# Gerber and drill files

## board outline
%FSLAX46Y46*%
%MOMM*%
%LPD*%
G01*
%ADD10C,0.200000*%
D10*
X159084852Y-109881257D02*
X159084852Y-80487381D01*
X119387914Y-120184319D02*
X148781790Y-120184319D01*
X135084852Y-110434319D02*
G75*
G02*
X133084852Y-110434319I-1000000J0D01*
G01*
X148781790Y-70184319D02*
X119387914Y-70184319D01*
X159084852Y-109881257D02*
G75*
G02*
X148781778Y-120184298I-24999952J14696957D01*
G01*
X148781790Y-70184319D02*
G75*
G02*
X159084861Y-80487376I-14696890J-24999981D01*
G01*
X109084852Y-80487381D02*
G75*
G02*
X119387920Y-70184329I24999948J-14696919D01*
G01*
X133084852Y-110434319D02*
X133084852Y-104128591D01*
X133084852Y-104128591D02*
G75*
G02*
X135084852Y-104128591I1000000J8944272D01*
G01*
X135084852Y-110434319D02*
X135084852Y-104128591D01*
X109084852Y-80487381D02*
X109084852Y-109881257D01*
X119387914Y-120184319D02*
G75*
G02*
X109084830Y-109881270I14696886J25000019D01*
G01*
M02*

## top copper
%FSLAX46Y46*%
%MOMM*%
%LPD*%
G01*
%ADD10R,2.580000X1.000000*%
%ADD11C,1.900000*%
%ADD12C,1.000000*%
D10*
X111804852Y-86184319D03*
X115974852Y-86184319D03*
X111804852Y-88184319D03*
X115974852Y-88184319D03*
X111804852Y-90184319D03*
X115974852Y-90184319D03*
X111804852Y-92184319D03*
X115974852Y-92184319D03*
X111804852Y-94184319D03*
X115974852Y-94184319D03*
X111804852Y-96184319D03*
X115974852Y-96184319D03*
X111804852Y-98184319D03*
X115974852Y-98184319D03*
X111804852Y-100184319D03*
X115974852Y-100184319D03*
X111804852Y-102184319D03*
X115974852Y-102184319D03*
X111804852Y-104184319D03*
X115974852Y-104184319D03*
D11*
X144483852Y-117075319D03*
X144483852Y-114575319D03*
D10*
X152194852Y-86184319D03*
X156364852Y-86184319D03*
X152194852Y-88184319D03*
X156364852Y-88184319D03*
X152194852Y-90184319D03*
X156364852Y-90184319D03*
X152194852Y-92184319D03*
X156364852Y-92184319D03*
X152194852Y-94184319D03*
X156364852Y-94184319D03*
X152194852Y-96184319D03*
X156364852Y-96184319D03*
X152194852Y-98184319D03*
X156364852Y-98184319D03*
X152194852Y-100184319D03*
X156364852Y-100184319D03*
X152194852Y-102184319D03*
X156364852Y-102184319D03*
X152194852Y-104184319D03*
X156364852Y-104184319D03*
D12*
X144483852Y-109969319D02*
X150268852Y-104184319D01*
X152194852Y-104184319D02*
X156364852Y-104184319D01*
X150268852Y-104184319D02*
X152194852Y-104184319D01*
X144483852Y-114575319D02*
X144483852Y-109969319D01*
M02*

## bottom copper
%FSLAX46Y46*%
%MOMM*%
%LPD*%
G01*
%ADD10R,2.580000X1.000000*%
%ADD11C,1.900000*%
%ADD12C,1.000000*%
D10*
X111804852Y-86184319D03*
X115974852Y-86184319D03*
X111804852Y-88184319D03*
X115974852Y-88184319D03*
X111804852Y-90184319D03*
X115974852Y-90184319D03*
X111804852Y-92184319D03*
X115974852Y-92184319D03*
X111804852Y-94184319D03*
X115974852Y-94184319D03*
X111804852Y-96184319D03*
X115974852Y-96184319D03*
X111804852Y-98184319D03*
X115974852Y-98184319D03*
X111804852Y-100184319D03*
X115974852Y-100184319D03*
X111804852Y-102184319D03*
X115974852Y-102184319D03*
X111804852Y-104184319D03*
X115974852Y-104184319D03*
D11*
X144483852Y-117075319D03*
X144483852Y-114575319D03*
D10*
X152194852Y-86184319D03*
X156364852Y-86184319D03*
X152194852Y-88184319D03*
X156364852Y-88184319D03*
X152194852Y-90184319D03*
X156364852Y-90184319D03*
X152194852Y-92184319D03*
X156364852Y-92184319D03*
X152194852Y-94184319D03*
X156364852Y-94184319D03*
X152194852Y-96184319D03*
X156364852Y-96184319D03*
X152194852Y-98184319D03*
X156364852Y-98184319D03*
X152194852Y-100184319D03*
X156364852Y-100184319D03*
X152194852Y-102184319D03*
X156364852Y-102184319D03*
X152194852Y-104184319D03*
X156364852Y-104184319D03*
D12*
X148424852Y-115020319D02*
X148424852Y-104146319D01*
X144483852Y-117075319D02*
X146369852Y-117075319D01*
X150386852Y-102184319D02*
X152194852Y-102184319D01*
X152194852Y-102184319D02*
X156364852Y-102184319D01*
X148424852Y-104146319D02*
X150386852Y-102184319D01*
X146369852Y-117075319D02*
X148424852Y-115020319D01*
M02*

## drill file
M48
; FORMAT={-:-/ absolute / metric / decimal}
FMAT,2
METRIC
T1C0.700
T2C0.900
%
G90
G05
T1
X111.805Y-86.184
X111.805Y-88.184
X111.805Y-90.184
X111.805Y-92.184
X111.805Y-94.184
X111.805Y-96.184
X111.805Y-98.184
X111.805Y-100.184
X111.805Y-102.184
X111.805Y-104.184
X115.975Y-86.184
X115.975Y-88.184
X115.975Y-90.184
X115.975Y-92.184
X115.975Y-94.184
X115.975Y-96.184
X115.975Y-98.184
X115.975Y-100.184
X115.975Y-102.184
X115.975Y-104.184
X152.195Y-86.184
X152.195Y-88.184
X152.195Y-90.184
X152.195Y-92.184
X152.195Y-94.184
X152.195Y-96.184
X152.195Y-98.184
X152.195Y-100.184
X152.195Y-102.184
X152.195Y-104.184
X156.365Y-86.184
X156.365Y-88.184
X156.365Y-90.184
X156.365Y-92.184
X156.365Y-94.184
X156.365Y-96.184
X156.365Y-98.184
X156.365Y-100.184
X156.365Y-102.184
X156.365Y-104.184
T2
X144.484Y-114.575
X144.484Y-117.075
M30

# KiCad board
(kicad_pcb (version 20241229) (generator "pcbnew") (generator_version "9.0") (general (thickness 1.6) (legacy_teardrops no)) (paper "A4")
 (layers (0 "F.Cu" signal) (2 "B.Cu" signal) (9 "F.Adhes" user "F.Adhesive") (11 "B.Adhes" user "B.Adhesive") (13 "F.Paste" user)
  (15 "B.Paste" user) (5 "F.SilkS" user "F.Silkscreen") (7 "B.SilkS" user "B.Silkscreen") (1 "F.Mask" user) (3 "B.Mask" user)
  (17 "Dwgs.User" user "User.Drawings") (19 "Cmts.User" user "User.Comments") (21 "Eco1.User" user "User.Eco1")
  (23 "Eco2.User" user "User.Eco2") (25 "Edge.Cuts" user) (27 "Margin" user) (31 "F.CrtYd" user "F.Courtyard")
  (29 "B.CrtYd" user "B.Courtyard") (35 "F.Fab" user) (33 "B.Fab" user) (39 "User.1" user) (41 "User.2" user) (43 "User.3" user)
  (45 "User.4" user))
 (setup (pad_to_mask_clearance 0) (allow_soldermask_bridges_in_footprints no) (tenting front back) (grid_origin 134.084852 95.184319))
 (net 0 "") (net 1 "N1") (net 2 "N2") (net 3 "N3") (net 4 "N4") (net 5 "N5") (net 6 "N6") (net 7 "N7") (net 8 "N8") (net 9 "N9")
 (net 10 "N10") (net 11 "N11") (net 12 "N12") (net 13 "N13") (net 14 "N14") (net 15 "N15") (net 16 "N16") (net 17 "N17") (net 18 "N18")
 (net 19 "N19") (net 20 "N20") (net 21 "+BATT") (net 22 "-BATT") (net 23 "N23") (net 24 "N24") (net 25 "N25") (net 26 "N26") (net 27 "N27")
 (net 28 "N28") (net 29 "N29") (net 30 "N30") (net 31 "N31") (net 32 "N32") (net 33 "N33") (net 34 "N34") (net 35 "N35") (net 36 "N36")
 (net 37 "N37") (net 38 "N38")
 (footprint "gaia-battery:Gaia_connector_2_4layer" (layer "F.Cu") (at 113.889852 95.184319)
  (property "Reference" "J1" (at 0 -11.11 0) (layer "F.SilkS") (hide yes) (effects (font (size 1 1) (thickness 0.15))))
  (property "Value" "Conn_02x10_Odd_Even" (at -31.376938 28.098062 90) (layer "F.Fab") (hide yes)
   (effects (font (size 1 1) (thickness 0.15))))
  (pad "1" thru_hole rect (at -2.085 -9) (size 2.58 1) (drill 0.7) (layers "*.Cu" "*.Mask") (remove_unused_layers no) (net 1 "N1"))
  (pad "2" thru_hole rect (at 2.085 -9) (size 2.58 1) (drill 0.7) (layers "*.Cu" "*.Mask") (remove_unused_layers no) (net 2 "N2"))
  (pad "3" thru_hole rect (at -2.085 -7) (size 2.58 1) (drill 0.7) (layers "*.Cu" "*.Mask") (remove_unused_layers no) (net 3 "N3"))
  (pad "4" thru_hole rect (at 2.085 -7) (size 2.58 1) (drill 0.7) (layers "*.Cu" "*.Mask") (remove_unused_layers no) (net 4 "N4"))
  (pad "5" thru_hole rect (at -2.085 -5) (size 2.58 1) (drill 0.7) (layers "*.Cu" "*.Mask") (remove_unused_layers no) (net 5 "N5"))
  (pad "6" thru_hole rect (at 2.085 -5) (size 2.58 1) (drill 0.7) (layers "*.Cu" "*.Mask") (remove_unused_layers no) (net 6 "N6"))
  (pad "7" thru_hole rect (at -2.085 -3) (size 2.58 1) (drill 0.7) (layers "*.Cu" "*.Mask") (remove_unused_layers no) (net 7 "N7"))
  (pad "8" thru_hole rect (at 2.085 -3) (size 2.58 1) (drill 0.7) (layers "*.Cu" "*.Mask") (remove_unused_layers no) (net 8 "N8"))
  (pad "9" thru_hole rect (at -2.085 -1) (size 2.58 1) (drill 0.7) (layers "*.Cu" "*.Mask") (remove_unused_layers no) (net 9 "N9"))
  (pad "10" thru_hole rect (at 2.085 -1) (size 2.58 1) (drill 0.7) (layers "*.Cu" "*.Mask") (remove_unused_layers no) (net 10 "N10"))
  (pad "11" thru_hole rect (at -2.085 1) (size 2.58 1) (drill 0.7) (layers "*.Cu" "*.Mask") (remove_unused_layers no) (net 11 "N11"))
  (pad "12" thru_hole rect (at 2.085 1) (size 2.58 1) (drill 0.7) (layers "*.Cu" "*.Mask") (remove_unused_layers no) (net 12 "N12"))
  (pad "13" thru_hole rect (at -2.085 3) (size 2.58 1) (drill 0.7) (layers "*.Cu" "*.Mask") (remove_unused_layers no) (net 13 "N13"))
  (pad "14" thru_hole rect (at 2.085 3) (size 2.58 1) (drill 0.7) (layers "*.Cu" "*.Mask") (remove_unused_layers no) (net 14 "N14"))
  (pad "15" thru_hole rect (at -2.085 5) (size 2.58 1) (drill 0.7) (layers "*.Cu" "*.Mask") (remove_unused_layers no) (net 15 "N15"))
  (pad "16" thru_hole rect (at 2.085 5) (size 2.58 1) (drill 0.7) (layers "*.Cu" "*.Mask") (remove_unused_layers no) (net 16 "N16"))
  (pad "17" thru_hole rect (at -2.085 7) (size 2.58 1) (drill 0.7) (layers "*.Cu" "*.Mask") (remove_unused_layers no) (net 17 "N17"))
  (pad "18" thru_hole rect (at 2.085 7) (size 2.58 1) (drill 0.7) (layers "*.Cu" "*.Mask") (remove_unused_layers no) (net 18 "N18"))
  (pad "19" thru_hole rect (at -2.085 9) (size 2.58 1) (drill 0.7) (layers "*.Cu" "*.Mask") (remove_unused_layers no) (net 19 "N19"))
  (pad "20" thru_hole rect (at 2.085 9) (size 2.58 1) (drill 0.7) (layers "*.Cu" "*.Mask") (remove_unused_layers no) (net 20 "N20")))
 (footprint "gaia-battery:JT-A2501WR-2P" (layer "F.Cu") (at 144.483852 117.075319 90)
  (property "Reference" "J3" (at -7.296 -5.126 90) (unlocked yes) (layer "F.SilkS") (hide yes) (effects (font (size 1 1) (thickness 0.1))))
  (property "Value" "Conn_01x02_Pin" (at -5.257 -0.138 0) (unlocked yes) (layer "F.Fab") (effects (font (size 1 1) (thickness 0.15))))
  (pad "1" thru_hole circle (at 0 0 90) (size 1.9 1.9) (drill 0.9) (layers "*.Cu" "*.Mask") (remove_unused_layers no) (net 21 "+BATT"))
  (pad "2" thru_hole circle (at 2.5 0 90) (size 1.9 1.9) (drill 0.9) (layers "*.Cu" "*.Mask") (remove_unused_layers no) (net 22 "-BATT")))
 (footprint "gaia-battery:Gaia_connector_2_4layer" (layer "F.Cu") (at 154.279852 95.184319)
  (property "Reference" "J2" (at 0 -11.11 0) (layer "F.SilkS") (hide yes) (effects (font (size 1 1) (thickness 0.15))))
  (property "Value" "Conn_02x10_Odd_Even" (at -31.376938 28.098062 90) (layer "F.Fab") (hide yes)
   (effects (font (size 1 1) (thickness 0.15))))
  (pad "1" thru_hole rect (at -2.085 -9) (size 2.58 1) (drill 0.7) (layers "*.Cu" "*.Mask") (remove_unused_layers no) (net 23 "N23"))
  (pad "2" thru_hole rect (at 2.085 -9) (size 2.58 1) (drill 0.7) (layers "*.Cu" "*.Mask") (remove_unused_layers no) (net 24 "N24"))
  (pad "3" thru_hole rect (at -2.085 -7) (size 2.58 1) (drill 0.7) (layers "*.Cu" "*.Mask") (remove_unused_layers no) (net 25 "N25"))
  (pad "4" thru_hole rect (at 2.085 -7) (size 2.58 1) (drill 0.7) (layers "*.Cu" "*.Mask") (remove_unused_layers no) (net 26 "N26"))
  (pad "5" thru_hole rect (at -2.085 -5) (size 2.58 1) (drill 0.7) (layers "*.Cu" "*.Mask") (remove_unused_layers no) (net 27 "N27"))
  (pad "6" thru_hole rect (at 2.085 -5) (size 2.58 1) (drill 0.7) (layers "*.Cu" "*.Mask") (remove_unused_layers no) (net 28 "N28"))
  (pad "7" thru_hole rect (at -2.085 -3) (size 2.58 1) (drill 0.7) (layers "*.Cu" "*.Mask") (remove_unused_layers no) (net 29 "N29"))
  (pad "8" thru_hole rect (at 2.085 -3) (size 2.58 1) (drill 0.7) (layers "*.Cu" "*.Mask") (remove_unused_layers no) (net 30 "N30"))
  (pad "9" thru_hole rect (at -2.085 -1) (size 2.58 1) (drill 0.7) (layers "*.Cu" "*.Mask") (remove_unused_layers no) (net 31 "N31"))
  (pad "10" thru_hole rect (at 2.085 -1) (size 2.58 1) (drill 0.7) (layers "*.Cu" "*.Mask") (remove_unused_layers no) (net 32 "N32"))
  (pad "11" thru_hole rect (at -2.085 1) (size 2.58 1) (drill 0.7) (layers "*.Cu" "*.Mask") (remove_unused_layers no) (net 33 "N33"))
  (pad "12" thru_hole rect (at 2.085 1) (size 2.58 1) (drill 0.7) (layers "*.Cu" "*.Mask") (remove_unused_layers no) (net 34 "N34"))
  (pad "13" thru_hole rect (at -2.085 3) (size 2.58 1) (drill 0.7) (layers "*.Cu" "*.Mask") (remove_unused_layers no) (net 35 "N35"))
  (pad "14" thru_hole rect (at 2.085 3) (size 2.58 1) (drill 0.7) (layers "*.Cu" "*.Mask") (remove_unused_layers no) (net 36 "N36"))
  (pad "15" thru_hole rect (at -2.085 5) (size 2.58 1) (drill 0.7) (layers "*.Cu" "*.Mask") (remove_unused_layers no) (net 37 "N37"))
  (pad "16" thru_hole rect (at 2.085 5) (size 2.58 1) (drill 0.7) (layers "*.Cu" "*.Mask") (remove_unused_layers no) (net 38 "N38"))
  (pad "17" thru_hole rect (at -2.085 7) (size 2.58 1) (drill 0.7) (layers "*.Cu" "*.Mask") (remove_unused_layers no) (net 21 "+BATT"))
  (pad "18" thru_hole rect (at 2.085 7) (size 2.58 1) (drill 0.7) (layers "*.Cu" "*.Mask") (remove_unused_layers no) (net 21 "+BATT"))
  (pad "19" thru_hole rect (at -2.085 9) (size 2.58 1) (drill 0.7) (layers "*.Cu" "*.Mask") (remove_unused_layers no) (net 22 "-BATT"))
  (pad "20" thru_hole rect (at 2.085 9) (size 2.58 1) (drill 0.7) (layers "*.Cu" "*.Mask") (remove_unused_layers no) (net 22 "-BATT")))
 (gr_line (start 159.084852 109.881257) (end 159.084852 80.487381) (stroke (width 0.2) (type default)) (locked yes) (layer "Edge.Cuts"))
 (gr_line (start 119.387914 120.184319) (end 148.78179 120.184319) (stroke (width 0.2) (type default)) (layer "Edge.Cuts"))
 (gr_arc (start 135.084852 110.434319) (mid 134.084852 111.434319) (end 133.084852 110.434319) (stroke (width 0.2) (type default))
  (layer "Edge.Cuts"))
 (gr_line (start 148.78179 70.184319) (end 119.387914 70.184319) (stroke (width 0.2) (type default)) (locked yes) (layer "Edge.Cuts"))
 (gr_arc (start 159.084852 109.881257) (mid 154.590949 115.690416) (end 148.78179 120.184319) (stroke (width 0.2) (type default))
  (layer "Edge.Cuts"))
 (gr_arc (start 148.78179 70.184319) (mid 154.590949 74.678222) (end 159.084852 80.487381) (stroke (width 0.2) (type default))
  (layer "Edge.Cuts"))
 (gr_arc (start 109.084852 80.487381) (mid 113.578755 74.678222) (end 119.387914 70.184319) (stroke (width 0.2) (type default))
  (layer "Edge.Cuts"))
 (gr_line (start 133.084852 110.434319) (end 133.084852 104.128591) (stroke (width 0.2) (type default)) (layer "Edge.Cuts"))
 (gr_arc (start 133.084852 104.128591) (mid 134.084852 86.184319) (end 135.084852 104.128591) (stroke (width 0.2) (type default))
  (layer "Edge.Cuts"))
 (gr_line (start 135.084852 110.434319) (end 135.084852 104.128591) (stroke (width 0.2) (type default)) (layer "Edge.Cuts"))
 (gr_line (start 109.084852 80.487381) (end 109.084852 109.881257) (stroke (width 0.2) (type default)) (locked yes) (layer "Edge.Cuts"))
 (gr_arc (start 119.387914 120.184319) (mid 113.578755 115.690416) (end 109.084852 109.881257) (stroke (width 0.2) (type default))
  (layer "Edge.Cuts"))
 (segment (start 144.483852 109.969319) (end 150.268852 104.184319) (width 1) (layer "F.Cu") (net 22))
 (segment (start 152.194852 104.184319) (end 156.364852 104.184319) (width 1) (layer "F.Cu") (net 22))
 (segment (start 150.268852 104.184319) (end 152.194852 104.184319) (width 1) (layer "F.Cu") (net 22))
 (segment (start 144.483852 114.575319) (end 144.483852 109.969319) (width 1) (layer "F.Cu") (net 22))
 (segment (start 148.424852 115.020319) (end 148.424852 104.146319) (width 1) (layer "B.Cu") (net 21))
 (segment (start 144.483852 117.075319) (end 146.369852 117.075319) (width 1) (layer "B.Cu") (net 21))
 (segment (start 150.386852 102.184319) (end 152.194852 102.184319) (width 1) (layer "B.Cu") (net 21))
 (segment (start 152.194852 102.184319) (end 156.364852 102.184319) (width 1) (layer "B.Cu") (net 21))
 (segment (start 148.424852 104.146319) (end 150.386852 102.184319) (width 1) (layer "B.Cu") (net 21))
 (segment (start 146.369852 117.075319) (end 148.424852 115.020319) (width 1) (layer "B.Cu") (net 21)))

